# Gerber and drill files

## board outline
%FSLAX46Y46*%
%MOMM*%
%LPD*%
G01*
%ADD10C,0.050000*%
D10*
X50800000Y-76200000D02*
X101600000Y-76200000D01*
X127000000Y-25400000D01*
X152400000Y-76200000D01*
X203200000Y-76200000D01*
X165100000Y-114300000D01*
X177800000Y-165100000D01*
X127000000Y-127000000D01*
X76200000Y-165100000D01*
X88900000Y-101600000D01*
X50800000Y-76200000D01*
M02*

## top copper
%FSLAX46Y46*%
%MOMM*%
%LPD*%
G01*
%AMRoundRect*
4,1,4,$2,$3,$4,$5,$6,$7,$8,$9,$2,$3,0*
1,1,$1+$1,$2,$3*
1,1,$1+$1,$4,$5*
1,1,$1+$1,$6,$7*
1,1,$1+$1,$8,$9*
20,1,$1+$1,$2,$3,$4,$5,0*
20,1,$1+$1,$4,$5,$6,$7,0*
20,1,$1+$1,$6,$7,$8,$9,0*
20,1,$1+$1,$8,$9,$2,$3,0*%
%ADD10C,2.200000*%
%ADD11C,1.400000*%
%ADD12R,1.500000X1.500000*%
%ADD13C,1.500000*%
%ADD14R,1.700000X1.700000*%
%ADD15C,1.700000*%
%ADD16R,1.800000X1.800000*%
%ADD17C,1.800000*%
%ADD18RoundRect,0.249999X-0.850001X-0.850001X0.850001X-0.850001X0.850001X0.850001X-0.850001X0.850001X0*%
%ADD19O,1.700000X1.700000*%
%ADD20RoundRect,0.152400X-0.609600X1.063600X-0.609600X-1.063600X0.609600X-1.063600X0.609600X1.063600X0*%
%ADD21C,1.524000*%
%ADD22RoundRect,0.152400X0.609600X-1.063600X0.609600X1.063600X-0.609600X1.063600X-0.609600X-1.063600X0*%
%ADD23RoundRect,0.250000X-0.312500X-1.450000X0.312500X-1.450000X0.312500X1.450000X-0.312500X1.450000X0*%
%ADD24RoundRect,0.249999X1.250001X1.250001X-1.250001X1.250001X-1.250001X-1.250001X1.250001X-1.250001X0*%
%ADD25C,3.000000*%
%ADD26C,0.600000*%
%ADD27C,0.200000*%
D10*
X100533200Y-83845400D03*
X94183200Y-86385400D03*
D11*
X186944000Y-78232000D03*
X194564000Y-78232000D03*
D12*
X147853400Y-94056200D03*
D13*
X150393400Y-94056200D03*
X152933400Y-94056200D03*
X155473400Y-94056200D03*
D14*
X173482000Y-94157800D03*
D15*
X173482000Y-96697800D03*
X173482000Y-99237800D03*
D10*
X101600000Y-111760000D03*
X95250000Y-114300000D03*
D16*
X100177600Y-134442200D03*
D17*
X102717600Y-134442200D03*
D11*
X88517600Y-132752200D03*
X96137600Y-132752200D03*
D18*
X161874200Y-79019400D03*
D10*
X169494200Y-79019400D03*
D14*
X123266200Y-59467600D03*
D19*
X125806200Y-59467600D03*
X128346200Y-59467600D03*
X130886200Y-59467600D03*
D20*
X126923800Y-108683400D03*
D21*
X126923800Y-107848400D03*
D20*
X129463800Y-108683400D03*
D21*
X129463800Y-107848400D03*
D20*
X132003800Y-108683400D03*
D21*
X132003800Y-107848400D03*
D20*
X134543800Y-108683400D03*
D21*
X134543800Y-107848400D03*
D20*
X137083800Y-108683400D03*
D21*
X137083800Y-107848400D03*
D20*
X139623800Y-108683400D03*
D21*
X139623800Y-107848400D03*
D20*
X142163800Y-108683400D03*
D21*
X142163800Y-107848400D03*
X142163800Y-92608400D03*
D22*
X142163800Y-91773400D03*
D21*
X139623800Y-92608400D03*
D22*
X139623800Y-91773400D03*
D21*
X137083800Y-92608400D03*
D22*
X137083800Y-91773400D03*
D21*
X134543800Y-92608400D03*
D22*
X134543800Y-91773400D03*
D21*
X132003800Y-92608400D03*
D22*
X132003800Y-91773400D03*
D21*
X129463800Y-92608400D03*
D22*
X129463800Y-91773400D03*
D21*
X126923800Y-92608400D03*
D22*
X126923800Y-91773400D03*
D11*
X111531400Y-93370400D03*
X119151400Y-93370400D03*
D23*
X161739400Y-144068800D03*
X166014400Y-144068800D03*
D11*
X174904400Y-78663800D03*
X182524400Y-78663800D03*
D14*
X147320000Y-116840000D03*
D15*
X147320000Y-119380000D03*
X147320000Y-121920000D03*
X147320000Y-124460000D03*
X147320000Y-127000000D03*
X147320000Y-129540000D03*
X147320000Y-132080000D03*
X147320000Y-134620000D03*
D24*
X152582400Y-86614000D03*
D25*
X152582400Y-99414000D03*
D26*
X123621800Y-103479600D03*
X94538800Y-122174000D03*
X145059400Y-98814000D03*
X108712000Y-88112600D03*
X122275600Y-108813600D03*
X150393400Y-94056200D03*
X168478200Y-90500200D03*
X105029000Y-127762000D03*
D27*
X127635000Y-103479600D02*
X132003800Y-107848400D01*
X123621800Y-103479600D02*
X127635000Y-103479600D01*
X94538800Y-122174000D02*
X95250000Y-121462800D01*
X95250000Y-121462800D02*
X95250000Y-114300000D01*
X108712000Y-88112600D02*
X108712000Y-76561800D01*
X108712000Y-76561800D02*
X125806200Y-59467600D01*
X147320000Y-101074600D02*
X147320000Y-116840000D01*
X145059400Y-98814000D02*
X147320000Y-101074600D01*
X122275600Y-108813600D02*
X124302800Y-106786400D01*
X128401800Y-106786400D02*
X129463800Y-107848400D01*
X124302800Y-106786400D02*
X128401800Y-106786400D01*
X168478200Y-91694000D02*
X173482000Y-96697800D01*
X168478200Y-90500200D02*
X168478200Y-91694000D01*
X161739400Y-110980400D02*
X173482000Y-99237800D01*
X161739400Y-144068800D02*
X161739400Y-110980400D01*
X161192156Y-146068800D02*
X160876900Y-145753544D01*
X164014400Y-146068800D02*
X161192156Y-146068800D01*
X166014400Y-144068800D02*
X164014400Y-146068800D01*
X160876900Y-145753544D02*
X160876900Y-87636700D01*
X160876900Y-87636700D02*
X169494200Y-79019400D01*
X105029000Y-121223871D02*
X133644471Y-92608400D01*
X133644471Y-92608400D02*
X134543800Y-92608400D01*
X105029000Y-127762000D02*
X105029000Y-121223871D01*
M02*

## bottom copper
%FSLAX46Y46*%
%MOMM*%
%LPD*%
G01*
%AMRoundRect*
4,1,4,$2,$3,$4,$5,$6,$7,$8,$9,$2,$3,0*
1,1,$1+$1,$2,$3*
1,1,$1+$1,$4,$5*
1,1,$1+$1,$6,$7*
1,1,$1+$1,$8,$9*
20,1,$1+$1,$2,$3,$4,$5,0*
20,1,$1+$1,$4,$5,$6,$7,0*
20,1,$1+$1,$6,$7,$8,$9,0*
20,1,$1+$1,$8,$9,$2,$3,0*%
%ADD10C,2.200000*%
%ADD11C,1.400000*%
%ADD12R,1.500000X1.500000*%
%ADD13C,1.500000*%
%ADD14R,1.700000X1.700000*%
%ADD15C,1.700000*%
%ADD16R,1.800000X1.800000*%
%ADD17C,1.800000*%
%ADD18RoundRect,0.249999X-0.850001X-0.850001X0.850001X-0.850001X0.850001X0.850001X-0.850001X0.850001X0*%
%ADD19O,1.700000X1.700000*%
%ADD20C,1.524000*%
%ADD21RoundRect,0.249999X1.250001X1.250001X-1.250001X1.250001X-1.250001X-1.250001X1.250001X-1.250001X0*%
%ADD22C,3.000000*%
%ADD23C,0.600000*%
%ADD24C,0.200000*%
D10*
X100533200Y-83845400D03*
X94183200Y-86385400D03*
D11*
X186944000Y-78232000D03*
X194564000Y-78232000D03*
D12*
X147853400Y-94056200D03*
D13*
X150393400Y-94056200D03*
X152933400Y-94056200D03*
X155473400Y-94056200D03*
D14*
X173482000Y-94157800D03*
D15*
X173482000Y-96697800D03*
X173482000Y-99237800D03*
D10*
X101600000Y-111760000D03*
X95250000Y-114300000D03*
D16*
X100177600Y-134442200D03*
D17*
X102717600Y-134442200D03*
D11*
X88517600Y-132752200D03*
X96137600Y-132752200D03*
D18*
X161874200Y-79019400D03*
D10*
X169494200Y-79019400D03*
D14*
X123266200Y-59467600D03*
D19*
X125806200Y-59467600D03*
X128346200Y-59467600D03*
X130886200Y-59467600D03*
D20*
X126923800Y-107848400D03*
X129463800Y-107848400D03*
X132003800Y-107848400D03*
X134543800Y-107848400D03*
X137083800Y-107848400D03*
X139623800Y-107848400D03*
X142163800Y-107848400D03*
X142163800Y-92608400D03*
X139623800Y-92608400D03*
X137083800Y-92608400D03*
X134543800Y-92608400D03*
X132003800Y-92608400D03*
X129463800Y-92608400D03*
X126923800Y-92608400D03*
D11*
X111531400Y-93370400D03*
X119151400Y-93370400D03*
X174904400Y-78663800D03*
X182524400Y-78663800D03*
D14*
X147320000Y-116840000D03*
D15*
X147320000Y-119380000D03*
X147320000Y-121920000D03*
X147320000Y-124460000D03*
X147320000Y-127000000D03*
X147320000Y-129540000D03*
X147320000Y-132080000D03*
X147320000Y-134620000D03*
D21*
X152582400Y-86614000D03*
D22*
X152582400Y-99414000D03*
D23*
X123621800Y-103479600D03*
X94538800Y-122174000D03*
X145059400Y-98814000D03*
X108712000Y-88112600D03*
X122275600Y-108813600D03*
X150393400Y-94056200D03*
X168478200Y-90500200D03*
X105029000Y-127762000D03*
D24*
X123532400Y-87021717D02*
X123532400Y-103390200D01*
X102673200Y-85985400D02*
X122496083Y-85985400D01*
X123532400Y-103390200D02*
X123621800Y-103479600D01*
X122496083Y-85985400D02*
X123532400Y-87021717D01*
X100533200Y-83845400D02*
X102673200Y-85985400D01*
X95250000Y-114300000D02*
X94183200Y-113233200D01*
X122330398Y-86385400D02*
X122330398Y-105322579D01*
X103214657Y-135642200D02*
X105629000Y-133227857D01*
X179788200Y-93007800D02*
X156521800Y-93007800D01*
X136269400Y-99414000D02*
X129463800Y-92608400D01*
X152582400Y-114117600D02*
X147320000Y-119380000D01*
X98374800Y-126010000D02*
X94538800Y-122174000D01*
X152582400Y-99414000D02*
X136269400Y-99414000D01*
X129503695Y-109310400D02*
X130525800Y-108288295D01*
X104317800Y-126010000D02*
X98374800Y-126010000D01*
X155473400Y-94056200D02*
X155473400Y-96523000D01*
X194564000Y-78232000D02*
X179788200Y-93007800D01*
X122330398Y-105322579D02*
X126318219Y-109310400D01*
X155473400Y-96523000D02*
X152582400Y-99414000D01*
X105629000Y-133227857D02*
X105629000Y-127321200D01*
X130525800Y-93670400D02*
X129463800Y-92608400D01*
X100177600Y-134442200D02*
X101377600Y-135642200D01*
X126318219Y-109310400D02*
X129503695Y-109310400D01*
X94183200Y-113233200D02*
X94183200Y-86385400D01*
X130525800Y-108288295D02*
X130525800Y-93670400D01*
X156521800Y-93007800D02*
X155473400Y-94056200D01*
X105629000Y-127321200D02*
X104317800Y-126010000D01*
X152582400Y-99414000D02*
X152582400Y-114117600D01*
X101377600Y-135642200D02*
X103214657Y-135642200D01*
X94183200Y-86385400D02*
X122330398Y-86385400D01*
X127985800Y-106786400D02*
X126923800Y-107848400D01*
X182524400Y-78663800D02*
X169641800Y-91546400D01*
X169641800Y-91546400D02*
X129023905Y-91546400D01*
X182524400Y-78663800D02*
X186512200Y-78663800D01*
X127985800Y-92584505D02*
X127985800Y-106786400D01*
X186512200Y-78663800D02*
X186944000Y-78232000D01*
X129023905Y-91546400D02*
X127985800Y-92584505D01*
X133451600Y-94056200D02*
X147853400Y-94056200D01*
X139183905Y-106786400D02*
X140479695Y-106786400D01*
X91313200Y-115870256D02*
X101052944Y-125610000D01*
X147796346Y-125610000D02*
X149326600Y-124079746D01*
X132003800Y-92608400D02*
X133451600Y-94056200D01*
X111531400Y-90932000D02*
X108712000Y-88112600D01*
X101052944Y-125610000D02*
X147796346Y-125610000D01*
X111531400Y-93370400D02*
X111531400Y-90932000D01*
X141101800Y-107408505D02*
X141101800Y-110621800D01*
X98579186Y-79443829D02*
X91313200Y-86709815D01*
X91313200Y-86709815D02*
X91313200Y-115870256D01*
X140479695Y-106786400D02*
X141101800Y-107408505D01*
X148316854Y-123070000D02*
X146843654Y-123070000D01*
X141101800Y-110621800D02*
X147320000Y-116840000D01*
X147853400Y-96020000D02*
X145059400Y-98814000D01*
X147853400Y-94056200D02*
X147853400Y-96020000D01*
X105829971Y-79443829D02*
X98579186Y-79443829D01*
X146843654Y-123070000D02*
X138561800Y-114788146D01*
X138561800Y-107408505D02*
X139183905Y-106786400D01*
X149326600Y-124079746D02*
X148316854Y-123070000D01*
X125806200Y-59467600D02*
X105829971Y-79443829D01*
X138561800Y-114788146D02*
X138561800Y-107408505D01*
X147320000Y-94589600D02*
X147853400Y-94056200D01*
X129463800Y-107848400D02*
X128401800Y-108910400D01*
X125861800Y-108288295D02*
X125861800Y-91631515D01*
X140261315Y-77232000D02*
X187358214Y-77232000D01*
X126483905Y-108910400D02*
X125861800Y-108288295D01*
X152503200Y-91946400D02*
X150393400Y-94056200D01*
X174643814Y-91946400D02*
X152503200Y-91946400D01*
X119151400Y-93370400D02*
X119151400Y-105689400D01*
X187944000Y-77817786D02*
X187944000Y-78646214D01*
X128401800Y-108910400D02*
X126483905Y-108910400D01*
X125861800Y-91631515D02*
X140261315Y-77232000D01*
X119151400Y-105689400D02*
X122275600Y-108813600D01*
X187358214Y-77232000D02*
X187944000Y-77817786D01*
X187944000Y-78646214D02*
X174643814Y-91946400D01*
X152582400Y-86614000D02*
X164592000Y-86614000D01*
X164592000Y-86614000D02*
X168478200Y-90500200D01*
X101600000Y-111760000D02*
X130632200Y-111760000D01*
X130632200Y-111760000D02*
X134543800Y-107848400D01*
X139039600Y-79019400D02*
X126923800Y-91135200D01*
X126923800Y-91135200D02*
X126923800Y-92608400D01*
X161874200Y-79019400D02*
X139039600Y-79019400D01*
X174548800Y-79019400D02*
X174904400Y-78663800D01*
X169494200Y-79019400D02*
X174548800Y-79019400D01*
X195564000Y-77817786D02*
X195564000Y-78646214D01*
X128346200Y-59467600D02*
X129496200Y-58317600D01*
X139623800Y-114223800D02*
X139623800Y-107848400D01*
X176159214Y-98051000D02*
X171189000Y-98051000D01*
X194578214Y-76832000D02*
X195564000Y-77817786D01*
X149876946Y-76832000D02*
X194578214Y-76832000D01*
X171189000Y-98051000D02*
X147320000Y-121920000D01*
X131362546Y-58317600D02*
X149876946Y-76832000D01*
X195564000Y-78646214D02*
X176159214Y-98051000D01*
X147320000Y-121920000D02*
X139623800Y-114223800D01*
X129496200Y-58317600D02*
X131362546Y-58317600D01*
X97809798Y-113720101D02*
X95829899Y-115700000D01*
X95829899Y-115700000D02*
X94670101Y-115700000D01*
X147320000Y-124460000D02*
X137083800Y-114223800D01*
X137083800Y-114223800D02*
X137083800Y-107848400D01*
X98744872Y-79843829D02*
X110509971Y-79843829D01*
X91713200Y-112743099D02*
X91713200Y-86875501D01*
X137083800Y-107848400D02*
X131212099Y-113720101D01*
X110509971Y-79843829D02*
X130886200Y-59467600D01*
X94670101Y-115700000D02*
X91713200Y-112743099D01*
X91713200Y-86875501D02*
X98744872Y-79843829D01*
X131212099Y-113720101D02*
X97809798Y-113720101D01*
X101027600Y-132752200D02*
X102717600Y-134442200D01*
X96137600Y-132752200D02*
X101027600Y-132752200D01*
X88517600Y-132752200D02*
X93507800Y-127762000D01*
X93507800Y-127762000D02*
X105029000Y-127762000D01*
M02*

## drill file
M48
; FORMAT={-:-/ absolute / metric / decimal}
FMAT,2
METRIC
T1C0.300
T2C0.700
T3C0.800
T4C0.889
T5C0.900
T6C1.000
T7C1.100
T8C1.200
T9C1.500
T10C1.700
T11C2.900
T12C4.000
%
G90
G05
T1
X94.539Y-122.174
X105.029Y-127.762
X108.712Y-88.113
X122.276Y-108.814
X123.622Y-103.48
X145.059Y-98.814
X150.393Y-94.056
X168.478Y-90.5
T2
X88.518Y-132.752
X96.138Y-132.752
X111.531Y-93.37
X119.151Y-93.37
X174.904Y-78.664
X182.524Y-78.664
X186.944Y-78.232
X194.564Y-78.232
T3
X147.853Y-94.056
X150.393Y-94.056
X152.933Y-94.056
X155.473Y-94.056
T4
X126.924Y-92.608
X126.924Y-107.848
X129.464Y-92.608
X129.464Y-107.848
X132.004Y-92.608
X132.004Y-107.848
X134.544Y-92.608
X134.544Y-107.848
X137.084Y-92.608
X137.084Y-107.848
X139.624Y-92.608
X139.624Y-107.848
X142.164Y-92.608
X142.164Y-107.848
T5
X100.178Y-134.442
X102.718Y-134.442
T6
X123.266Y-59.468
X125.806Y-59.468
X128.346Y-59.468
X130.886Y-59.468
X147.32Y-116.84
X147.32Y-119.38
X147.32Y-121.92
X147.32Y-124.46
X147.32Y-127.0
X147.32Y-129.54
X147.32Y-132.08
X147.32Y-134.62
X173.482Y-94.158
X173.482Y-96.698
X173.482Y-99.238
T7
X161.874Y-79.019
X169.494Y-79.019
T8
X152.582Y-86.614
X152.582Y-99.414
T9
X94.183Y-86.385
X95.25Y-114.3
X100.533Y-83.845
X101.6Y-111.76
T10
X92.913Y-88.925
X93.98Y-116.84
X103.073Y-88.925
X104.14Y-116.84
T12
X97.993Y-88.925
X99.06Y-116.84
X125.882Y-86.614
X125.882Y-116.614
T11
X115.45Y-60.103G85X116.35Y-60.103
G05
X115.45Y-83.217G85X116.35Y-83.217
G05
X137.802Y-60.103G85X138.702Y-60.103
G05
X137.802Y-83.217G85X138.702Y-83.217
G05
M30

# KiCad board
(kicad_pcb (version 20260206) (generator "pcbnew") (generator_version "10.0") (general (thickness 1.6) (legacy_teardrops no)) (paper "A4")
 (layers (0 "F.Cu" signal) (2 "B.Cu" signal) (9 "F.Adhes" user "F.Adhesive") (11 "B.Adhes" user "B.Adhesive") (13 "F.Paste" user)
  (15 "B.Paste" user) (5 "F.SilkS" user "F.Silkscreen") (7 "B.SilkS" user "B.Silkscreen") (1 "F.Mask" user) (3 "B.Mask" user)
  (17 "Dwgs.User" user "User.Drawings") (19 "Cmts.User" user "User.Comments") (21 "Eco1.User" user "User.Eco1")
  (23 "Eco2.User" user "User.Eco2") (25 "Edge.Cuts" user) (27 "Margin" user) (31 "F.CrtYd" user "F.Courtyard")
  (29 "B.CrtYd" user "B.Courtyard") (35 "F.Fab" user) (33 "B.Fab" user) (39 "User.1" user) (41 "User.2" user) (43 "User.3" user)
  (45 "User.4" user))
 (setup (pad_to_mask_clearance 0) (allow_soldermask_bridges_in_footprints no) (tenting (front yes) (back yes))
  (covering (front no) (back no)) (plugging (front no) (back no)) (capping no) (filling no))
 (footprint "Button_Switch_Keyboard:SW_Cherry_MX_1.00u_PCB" (layer "F.Cu") (at 100.5332 83.8454)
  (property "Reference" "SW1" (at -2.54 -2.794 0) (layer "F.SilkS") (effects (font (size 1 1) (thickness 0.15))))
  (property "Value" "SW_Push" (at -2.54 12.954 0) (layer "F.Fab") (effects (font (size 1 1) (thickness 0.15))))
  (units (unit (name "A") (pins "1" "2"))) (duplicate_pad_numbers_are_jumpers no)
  (pad "" np_thru_hole circle (at -7.62 5.08) (size 1.7 1.7) (drill 1.7) (layers "*.Cu" "*.Mask"))
  (pad "" np_thru_hole circle (at -2.54 5.08) (size 4 4) (drill 4) (layers "*.Cu" "*.Mask"))
  (pad "" np_thru_hole circle (at 2.54 5.08) (size 1.7 1.7) (drill 1.7) (layers "*.Cu" "*.Mask"))
  (pad "1" thru_hole circle (at 0 0) (size 2.2 2.2) (drill 1.5) (layers "*.Cu" "*.Mask") (remove_unused_layers no) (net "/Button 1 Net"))
  (pad "2" thru_hole circle (at -6.35 2.54) (size 2.2 2.2) (drill 1.5) (layers "*.Cu" "*.Mask") (remove_unused_layers no) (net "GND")))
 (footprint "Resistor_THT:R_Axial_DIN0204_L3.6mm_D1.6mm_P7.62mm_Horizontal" (layer "F.Cu") (at 186.944 78.232)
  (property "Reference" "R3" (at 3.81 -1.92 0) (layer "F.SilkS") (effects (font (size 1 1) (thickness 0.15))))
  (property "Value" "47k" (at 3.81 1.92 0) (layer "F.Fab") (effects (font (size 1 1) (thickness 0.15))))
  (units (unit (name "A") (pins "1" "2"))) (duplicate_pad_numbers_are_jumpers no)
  (pad "1" thru_hole circle (at 0 0) (size 1.4 1.4) (drill 0.7) (layers "*.Cu" "*.Mask") (remove_unused_layers no) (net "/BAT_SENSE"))
  (pad "2" thru_hole circle (at 7.62 0) (size 1.4 1.4) (drill 0.7) (layers "*.Cu" "*.Mask") (remove_unused_layers no) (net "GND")))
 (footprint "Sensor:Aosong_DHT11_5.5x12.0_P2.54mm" (layer "F.Cu") (at 147.8534 94.0562 90)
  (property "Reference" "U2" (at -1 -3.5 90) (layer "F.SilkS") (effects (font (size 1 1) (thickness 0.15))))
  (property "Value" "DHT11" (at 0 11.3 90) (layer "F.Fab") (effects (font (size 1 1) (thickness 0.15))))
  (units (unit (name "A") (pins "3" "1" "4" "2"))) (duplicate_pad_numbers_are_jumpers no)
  (pad "1" thru_hole rect (at 0 0 90) (size 1.5 1.5) (drill 0.8) (layers "*.Cu" "*.Mask") (remove_unused_layers no) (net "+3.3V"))
  (pad "2" thru_hole circle (at 0 2.54 90) (size 1.5 1.5) (drill 0.8) (layers "*.Cu" "*.Mask") (remove_unused_layers no) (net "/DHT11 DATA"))
  (pad "3" thru_hole circle (at 0 5.08 90) (size 1.5 1.5) (drill 0.8) (layers "*.Cu" "*.Mask") (remove_unused_layers no)
   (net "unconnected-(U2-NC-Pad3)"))
  (pad "4" thru_hole circle (at 0 7.62 90) (size 1.5 1.5) (drill 0.8) (layers "*.Cu" "*.Mask") (remove_unused_layers no) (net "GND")))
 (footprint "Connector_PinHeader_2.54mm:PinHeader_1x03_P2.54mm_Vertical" (layer "F.Cu") (at 173.482 94.1578)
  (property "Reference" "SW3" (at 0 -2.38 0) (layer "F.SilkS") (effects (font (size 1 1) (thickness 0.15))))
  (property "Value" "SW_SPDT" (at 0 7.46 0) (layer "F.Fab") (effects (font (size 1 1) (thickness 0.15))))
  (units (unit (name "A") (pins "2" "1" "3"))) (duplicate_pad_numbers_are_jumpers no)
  (pad "1" thru_hole rect (at 0 0) (size 1.7 1.7) (drill 1) (layers "*.Cu" "*.Mask") (remove_unused_layers no)
   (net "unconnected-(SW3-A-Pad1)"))
  (pad "2" thru_hole circle (at 0 2.54) (size 1.7 1.7) (drill 1) (layers "*.Cu" "*.Mask") (remove_unused_layers no) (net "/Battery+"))
  (pad "3" thru_hole circle (at 0 5.08) (size 1.7 1.7) (drill 1) (layers "*.Cu" "*.Mask") (remove_unused_layers no) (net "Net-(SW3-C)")))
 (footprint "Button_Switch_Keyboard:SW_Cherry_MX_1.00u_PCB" (layer "F.Cu") (at 101.6 111.76)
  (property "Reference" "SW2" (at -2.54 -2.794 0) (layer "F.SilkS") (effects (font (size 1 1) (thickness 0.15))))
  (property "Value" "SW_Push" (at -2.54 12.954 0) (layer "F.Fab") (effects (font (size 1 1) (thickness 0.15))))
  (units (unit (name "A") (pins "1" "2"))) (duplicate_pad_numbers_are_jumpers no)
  (pad "" np_thru_hole circle (at -7.62 5.08) (size 1.7 1.7) (drill 1.7) (layers "*.Cu" "*.Mask"))
  (pad "" np_thru_hole circle (at -2.54 5.08) (size 4 4) (drill 4) (layers "*.Cu" "*.Mask"))
  (pad "" np_thru_hole circle (at 2.54 5.08) (size 1.7 1.7) (drill 1.7) (layers "*.Cu" "*.Mask"))
  (pad "1" thru_hole circle (at 0 0) (size 2.2 2.2) (drill 1.5) (layers "*.Cu" "*.Mask") (remove_unused_layers no) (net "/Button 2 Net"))
  (pad "2" thru_hole circle (at -6.35 2.54) (size 2.2 2.2) (drill 1.5) (layers "*.Cu" "*.Mask") (remove_unused_layers no) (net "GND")))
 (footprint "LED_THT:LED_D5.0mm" (layer "F.Cu") (at 100.1776 134.4422)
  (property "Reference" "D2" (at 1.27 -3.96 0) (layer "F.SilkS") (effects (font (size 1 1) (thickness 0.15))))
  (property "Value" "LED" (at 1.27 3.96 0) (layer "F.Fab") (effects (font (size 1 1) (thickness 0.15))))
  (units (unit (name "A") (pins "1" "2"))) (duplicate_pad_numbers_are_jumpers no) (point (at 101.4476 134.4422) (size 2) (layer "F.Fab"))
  (pad "1" thru_hole rect (at 0 0) (size 1.8 1.8) (drill 0.9) (layers "*.Cu" "*.Mask") (remove_unused_layers no) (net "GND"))
  (pad "2" thru_hole circle (at 2.54 0) (size 1.8 1.8) (drill 0.9) (layers "*.Cu" "*.Mask") (remove_unused_layers no) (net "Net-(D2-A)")))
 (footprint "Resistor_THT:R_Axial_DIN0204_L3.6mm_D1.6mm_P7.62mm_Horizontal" (layer "F.Cu") (at 88.5176 132.7522)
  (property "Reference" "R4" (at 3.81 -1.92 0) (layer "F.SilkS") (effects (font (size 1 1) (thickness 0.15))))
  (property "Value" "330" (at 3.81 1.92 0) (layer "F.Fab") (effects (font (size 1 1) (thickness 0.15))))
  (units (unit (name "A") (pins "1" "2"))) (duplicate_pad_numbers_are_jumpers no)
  (pad "1" thru_hole circle (at 0 0) (size 1.4 1.4) (drill 0.7) (layers "*.Cu" "*.Mask") (remove_unused_layers no) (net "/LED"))
  (pad "2" thru_hole circle (at 7.62 0) (size 1.4 1.4) (drill 0.7) (layers "*.Cu" "*.Mask") (remove_unused_layers no) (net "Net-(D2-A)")))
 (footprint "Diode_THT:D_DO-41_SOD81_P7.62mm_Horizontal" (layer "F.Cu") (at 161.8742 79.0194)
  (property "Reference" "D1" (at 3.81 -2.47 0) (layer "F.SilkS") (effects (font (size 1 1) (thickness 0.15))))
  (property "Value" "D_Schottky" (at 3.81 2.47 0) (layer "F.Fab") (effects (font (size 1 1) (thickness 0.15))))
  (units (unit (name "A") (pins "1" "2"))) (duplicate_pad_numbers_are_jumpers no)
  (pad "1" thru_hole roundrect (at 0 0) (size 2.2 2.2) (drill 1.1) (layers "*.Cu" "*.Mask") (remove_unused_layers no)
   (roundrect_rratio 0.113636) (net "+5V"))
  (pad "2" thru_hole circle (at 7.62 0) (size 2.2 2.2) (drill 1.1) (layers "*.Cu" "*.Mask") (remove_unused_layers no) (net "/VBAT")))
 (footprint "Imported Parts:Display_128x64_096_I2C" (layer "F.Cu") (at 127.0762 59.4676)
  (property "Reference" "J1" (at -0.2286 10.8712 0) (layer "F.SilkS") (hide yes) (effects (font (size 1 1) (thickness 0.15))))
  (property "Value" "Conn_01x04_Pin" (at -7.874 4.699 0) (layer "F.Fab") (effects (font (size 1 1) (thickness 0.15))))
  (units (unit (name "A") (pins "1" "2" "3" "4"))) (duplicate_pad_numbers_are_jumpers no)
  (pad "" np_thru_hole oval (at -11.176 0.635) (size 3.8 2.9) (drill oval 3.8 2.9) (layers "*.Cu" "*.Mask"))
  (pad "" np_thru_hole oval (at -11.176 23.749) (size 3.8 2.9) (drill oval 3.8 2.9) (layers "*.Cu" "*.Mask"))
  (pad "" np_thru_hole oval (at 11.176 0.635) (size 3.8 2.9) (drill oval 3.8 2.9) (layers "*.Cu" "*.Mask"))
  (pad "" np_thru_hole oval (at 11.176 23.749) (size 3.8 2.9) (drill oval 3.8 2.9) (layers "*.Cu" "*.Mask"))
  (pad "1" thru_hole rect (at -3.81 0 90) (size 1.7 1.7) (drill 1) (layers "*.Cu" "*.Mask") (remove_unused_layers no) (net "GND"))
  (pad "2" thru_hole oval (at -1.27 0 90) (size 1.7 1.7) (drill 1) (layers "*.Cu" "*.Mask") (remove_unused_layers no) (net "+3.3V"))
  (pad "3" thru_hole oval (at 1.27 0 90) (size 1.7 1.7) (drill 1) (layers "*.Cu" "*.Mask") (remove_unused_layers no) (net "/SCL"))
  (pad "4" thru_hole oval (at 3.81 0 90) (size 1.7 1.7) (drill 1) (layers "*.Cu" "*.Mask") (remove_unused_layers no) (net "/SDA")))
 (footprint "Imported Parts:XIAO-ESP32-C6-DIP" (layer "F.Cu") (at 134.5438 100.2284 180)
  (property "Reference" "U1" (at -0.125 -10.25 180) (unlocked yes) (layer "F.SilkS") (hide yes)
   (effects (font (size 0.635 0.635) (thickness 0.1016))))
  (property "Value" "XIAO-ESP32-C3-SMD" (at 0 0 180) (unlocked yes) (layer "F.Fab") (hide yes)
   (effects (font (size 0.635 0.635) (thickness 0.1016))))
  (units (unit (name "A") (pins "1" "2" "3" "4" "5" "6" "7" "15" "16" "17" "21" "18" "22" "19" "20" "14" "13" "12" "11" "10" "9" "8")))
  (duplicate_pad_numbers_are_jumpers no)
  (pad "1" smd roundrect (at 7.62 -8.455 270) (size 2.432 1.524) (layers "F.Cu" "F.Mask") (roundrect_rratio 0.1) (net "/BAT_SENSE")
   (thermal_bridge_angle 45))
  (pad "1" thru_hole circle (at 7.62 -7.62 270) (size 1.524 1.524) (drill 0.889) (layers "*.Cu" "*.Mask") (remove_unused_layers no)
   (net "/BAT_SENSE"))
  (pad "2" smd roundrect (at 5.08 -8.455 270) (size 2.432 1.524) (layers "F.Cu" "F.Mask") (roundrect_rratio 0.1) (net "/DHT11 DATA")
   (thermal_bridge_angle 45))
  (pad "2" thru_hole circle (at 5.08 -7.62 270) (size 1.524 1.524) (drill 0.889) (layers "*.Cu" "*.Mask") (remove_unused_layers no)
   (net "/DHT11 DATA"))
  (pad "3" smd roundrect (at 2.54 -8.455 270) (size 2.432 1.524) (layers "F.Cu" "F.Mask") (roundrect_rratio 0.1) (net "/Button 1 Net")
   (thermal_bridge_angle 45))
  (pad "3" thru_hole circle (at 2.54 -7.62 270) (size 1.524 1.524) (drill 0.889) (layers "*.Cu" "*.Mask") (remove_unused_layers no)
   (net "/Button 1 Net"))
  (pad "4" smd roundrect (at 0 -8.455 270) (size 2.432 1.524) (layers "F.Cu" "F.Mask") (roundrect_rratio 0.1) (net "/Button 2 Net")
   (thermal_bridge_angle 45))
  (pad "4" thru_hole circle (at 0 -7.62 270) (size 1.524 1.524) (drill 0.889) (layers "*.Cu" "*.Mask") (remove_unused_layers no)
   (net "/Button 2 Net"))
  (pad "5" smd roundrect (at -2.54 -8.455 270) (size 2.432 1.524) (layers "F.Cu" "F.Mask") (roundrect_rratio 0.1) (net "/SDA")
   (thermal_bridge_angle 45))
  (pad "5" thru_hole circle (at -2.54 -7.62 270) (size 1.524 1.524) (drill 0.889) (layers "*.Cu" "*.Mask") (remove_unused_layers no)
   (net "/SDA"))
  (pad "6" smd roundrect (at -5.08 -8.455 270) (size 2.432 1.524) (layers "F.Cu" "F.Mask") (roundrect_rratio 0.1) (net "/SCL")
   (thermal_bridge_angle 45))
  (pad "6" thru_hole circle (at -5.08 -7.62 270) (size 1.524 1.524) (drill 0.889) (layers "*.Cu" "*.Mask") (remove_unused_layers no)
   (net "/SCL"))
  (pad "7" smd roundrect (at -7.62 -8.455 270) (size 2.432 1.524) (layers "F.Cu" "F.Mask") (roundrect_rratio 0.1)
   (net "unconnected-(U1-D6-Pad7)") (thermal_bridge_angle 45))
  (pad "7" thru_hole circle (at -7.62 -7.62 270) (size 1.524 1.524) (drill 0.889) (layers "*.Cu" "*.Mask") (remove_unused_layers no)
   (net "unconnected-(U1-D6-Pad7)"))
  (pad "8" thru_hole circle (at -7.62 7.62 90) (size 1.524 1.524) (drill 0.889) (layers "*.Cu" "*.Mask") (remove_unused_layers no)
   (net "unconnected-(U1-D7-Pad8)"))
  (pad "8" smd roundrect (at -7.62 8.455 90) (size 2.432 1.524) (layers "F.Cu" "F.Mask") (roundrect_rratio 0.1)
   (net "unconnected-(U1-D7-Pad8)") (thermal_bridge_angle 45))
  (pad "9" thru_hole circle (at -5.08 7.62 90) (size 1.524 1.524) (drill 0.889) (layers "*.Cu" "*.Mask") (remove_unused_layers no)
   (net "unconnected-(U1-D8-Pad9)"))
  (pad "9" smd roundrect (at -5.08 8.455 90) (size 2.432 1.524) (layers "F.Cu" "F.Mask") (roundrect_rratio 0.1)
   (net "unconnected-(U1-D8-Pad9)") (thermal_bridge_angle 45))
  (pad "10" thru_hole circle (at -2.54 7.62 90) (size 1.524 1.524) (drill 0.889) (layers "*.Cu" "*.Mask") (remove_unused_layers no)
   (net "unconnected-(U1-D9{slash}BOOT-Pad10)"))
  (pad "10" smd roundrect (at -2.54 8.455 90) (size 2.432 1.524) (layers "F.Cu" "F.Mask") (roundrect_rratio 0.1)
   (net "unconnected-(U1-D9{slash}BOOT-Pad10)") (thermal_bridge_angle 45))
  (pad "11" thru_hole circle (at 0 7.62 90) (size 1.524 1.524) (drill 0.889) (layers "*.Cu" "*.Mask") (remove_unused_layers no) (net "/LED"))
  (pad "11" smd roundrect (at 0 8.455 90) (size 2.432 1.524) (layers "F.Cu" "F.Mask") (roundrect_rratio 0.1) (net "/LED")
   (thermal_bridge_angle 45))
  (pad "12" thru_hole circle (at 2.54 7.62 90) (size 1.524 1.524) (drill 0.889) (layers "*.Cu" "*.Mask") (remove_unused_layers no)
   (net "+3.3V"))
  (pad "12" smd roundrect (at 2.54 8.455 90) (size 2.432 1.524) (layers "F.Cu" "F.Mask") (roundrect_rratio 0.1) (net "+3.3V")
   (thermal_bridge_angle 45))
  (pad "13" thru_hole circle (at 5.08 7.62 90) (size 1.524 1.524) (drill 0.889) (layers "*.Cu" "*.Mask") (remove_unused_layers no)
   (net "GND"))
  (pad "13" smd roundrect (at 5.08 8.455 90) (size 2.432 1.524) (layers "F.Cu" "F.Mask") (roundrect_rratio 0.1) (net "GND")
   (thermal_bridge_angle 45))
  (pad "14" thru_hole circle (at 7.62 7.62 90) (size 1.524 1.524) (drill 0.889) (layers "*.Cu" "*.Mask") (remove_unused_layers no)
   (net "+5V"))
  (pad "14" smd roundrect (at 7.62 8.455 90) (size 2.432 1.524) (layers "F.Cu" "F.Mask") (roundrect_rratio 0.1) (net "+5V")
   (thermal_bridge_angle 45)))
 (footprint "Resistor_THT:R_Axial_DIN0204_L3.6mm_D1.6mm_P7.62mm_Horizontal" (layer "F.Cu") (at 111.5314 93.3704)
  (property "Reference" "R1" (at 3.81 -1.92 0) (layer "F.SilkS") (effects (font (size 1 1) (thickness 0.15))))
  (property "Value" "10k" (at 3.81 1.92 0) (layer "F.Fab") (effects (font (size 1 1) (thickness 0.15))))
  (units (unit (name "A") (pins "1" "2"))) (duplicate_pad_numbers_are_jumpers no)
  (pad "1" thru_hole circle (at 0 0) (size 1.4 1.4) (drill 0.7) (layers "*.Cu" "*.Mask") (remove_unused_layers no) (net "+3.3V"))
  (pad "2" thru_hole circle (at 7.62 0) (size 1.4 1.4) (drill 0.7) (layers "*.Cu" "*.Mask") (remove_unused_layers no) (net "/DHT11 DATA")))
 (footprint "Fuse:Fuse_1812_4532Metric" (layer "F.Cu") (at 163.8769 144.0688)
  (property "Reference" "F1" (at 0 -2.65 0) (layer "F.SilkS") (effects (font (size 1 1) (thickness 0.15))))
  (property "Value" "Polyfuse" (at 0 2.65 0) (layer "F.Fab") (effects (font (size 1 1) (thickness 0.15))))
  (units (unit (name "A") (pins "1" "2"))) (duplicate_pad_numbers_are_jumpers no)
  (pad "1" smd roundrect (at -2.1375 0) (size 1.125 3.4) (layers "F.Cu" "F.Mask" "F.Paste") (roundrect_rratio 0.222222) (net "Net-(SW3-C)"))
  (pad "2" smd roundrect (at 2.1375 0) (size 1.125 3.4) (layers "F.Cu" "F.Mask" "F.Paste") (roundrect_rratio 0.222222) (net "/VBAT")))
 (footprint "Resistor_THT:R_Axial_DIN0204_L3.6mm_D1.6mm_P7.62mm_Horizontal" (layer "F.Cu") (at 174.9044 78.6638)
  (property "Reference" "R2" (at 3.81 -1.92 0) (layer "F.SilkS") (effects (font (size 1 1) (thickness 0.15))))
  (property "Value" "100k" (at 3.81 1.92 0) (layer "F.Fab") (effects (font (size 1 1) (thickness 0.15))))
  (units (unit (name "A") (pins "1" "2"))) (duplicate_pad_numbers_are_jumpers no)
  (pad "1" thru_hole circle (at 0 0) (size 1.4 1.4) (drill 0.7) (layers "*.Cu" "*.Mask") (remove_unused_layers no) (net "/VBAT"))
  (pad "2" thru_hole circle (at 7.62 0) (size 1.4 1.4) (drill 0.7) (layers "*.Cu" "*.Mask") (remove_unused_layers no) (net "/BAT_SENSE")))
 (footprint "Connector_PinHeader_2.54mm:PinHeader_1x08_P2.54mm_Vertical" (layer "F.Cu") (at 147.32 116.84)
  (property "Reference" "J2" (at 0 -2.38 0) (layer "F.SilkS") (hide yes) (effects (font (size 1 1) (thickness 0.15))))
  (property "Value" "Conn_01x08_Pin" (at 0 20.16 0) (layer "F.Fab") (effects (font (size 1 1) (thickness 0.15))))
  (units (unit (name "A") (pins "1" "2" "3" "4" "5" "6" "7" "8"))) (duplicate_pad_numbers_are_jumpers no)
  (pad "1" thru_hole rect (at 0 0) (size 1.7 1.7) (drill 1) (layers "*.Cu" "*.Mask") (remove_unused_layers no) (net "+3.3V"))
  (pad "2" thru_hole circle (at 0 2.54) (size 1.7 1.7) (drill 1) (layers "*.Cu" "*.Mask") (remove_unused_layers no) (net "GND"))
  (pad "3" thru_hole circle (at 0 5.08) (size 1.7 1.7) (drill 1) (layers "*.Cu" "*.Mask") (remove_unused_layers no) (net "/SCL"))
  (pad "4" thru_hole circle (at 0 7.62) (size 1.7 1.7) (drill 1) (layers "*.Cu" "*.Mask") (remove_unused_layers no) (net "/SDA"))
  (pad "5" thru_hole circle (at 0 10.16) (size 1.7 1.7) (drill 1) (layers "*.Cu" "*.Mask") (remove_unused_layers no)
   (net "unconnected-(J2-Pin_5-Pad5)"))
  (pad "6" thru_hole circle (at 0 12.7) (size 1.7 1.7) (drill 1) (layers "*.Cu" "*.Mask") (remove_unused_layers no)
   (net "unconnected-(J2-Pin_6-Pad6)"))
  (pad "7" thru_hole circle (at 0 15.24) (size 1.7 1.7) (drill 1) (layers "*.Cu" "*.Mask") (remove_unused_layers no)
   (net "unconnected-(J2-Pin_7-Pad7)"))
  (pad "8" thru_hole circle (at 0 17.78) (size 1.7 1.7) (drill 1) (layers "*.Cu" "*.Mask") (remove_unused_layers no)
   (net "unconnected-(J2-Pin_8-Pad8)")))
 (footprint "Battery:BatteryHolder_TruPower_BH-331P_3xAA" (layer "B.Cu") (at 152.5824 86.614 180)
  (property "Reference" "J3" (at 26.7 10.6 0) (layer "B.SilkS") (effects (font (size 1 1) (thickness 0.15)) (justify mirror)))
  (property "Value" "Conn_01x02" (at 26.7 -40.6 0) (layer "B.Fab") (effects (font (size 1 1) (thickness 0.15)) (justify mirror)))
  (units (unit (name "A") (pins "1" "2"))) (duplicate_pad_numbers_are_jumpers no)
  (pad "" np_thru_hole circle (at 26.7 -30 180) (size 4 4) (drill 4) (layers "*.Cu" "*.Mask"))
  (pad "" np_thru_hole circle (at 26.7 0 180) (size 4 4) (drill 4) (layers "*.Cu" "*.Mask"))
  (pad "1" thru_hole roundrect (at 0 0 180) (size 3 3) (drill 1.2) (layers "*.Cu" "*.Mask") (remove_unused_layers no)
   (roundrect_rratio 0.083333) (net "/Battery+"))
  (pad "2" thru_hole circle (at 0 -12.8 180) (size 3 3) (drill 1.2) (layers "*.Cu" "*.Mask") (remove_unused_layers no) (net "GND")))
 (gr_poly
  (pts (xy 50.8 76.2) (xy 101.6 76.2) (xy 127 25.4) (xy 152.4 76.2) (xy 203.2 76.2) (xy 165.1 114.3) (xy 177.8 165.1) (xy 127 127)
   (xy 76.2 165.1) (xy 88.9 101.6))
  (stroke (width 0.05) (type solid)) (fill no) (layer "Edge.Cuts"))
 (segment (start 127.635 103.4796) (end 132.0038 107.8484) (width 0.2) (layer "F.Cu") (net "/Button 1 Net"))
 (segment (start 123.6218 103.4796) (end 127.635 103.4796) (width 0.2) (layer "F.Cu") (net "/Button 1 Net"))
 (via (at 123.6218 103.4796) (size 0.6) (drill 0.3) (layers "F.Cu" "B.Cu") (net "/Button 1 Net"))
 (segment (start 123.5324 87.021717) (end 123.5324 103.3902) (width 0.2) (layer "B.Cu") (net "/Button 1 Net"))
 (segment (start 102.6732 85.9854) (end 122.496083 85.9854) (width 0.2) (layer "B.Cu") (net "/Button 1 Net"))
 (segment (start 123.5324 103.3902) (end 123.6218 103.4796) (width 0.2) (layer "B.Cu") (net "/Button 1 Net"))
 (segment (start 122.496083 85.9854) (end 123.5324 87.021717) (width 0.2) (layer "B.Cu") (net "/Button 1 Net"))
 (segment (start 100.5332 83.8454) (end 102.6732 85.9854) (width 0.2) (layer "B.Cu") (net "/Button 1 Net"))
 (segment (start 94.5388 122.174) (end 95.25 121.4628) (width 0.2) (layer "F.Cu") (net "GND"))
 (segment (start 95.25 121.4628) (end 95.25 114.3) (width 0.2) (layer "F.Cu") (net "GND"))
 (via (at 94.5388 122.174) (size 0.6) (drill 0.3) (layers "F.Cu" "B.Cu") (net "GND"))
 (segment (start 95.25 114.3) (end 94.1832 113.2332) (width 0.2) (layer "B.Cu") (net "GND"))
 (segment (start 122.330398 86.3854) (end 122.330398 105.322579) (width 0.2) (layer "B.Cu") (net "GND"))
 (segment (start 103.214657 135.6422) (end 105.629 133.227857) (width 0.2) (layer "B.Cu") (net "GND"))
 (segment (start 179.7882 93.0078) (end 156.5218 93.0078) (width 0.2) (layer "B.Cu") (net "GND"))
 (segment (start 136.2694 99.414) (end 129.4638 92.6084) (width 0.2) (layer "B.Cu") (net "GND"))
 (segment (start 152.5824 114.1176) (end 147.32 119.38) (width 0.2) (layer "B.Cu") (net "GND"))
 (segment (start 98.3748 126.01) (end 94.5388 122.174) (width 0.2) (layer "B.Cu") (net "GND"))
 (segment (start 152.5824 99.414) (end 136.2694 99.414) (width 0.2) (layer "B.Cu") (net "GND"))
 (segment (start 129.503695 109.3104) (end 130.5258 108.288295) (width 0.2) (layer "B.Cu") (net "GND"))
 (segment (start 104.3178 126.01) (end 98.3748 126.01) (width 0.2) (layer "B.Cu") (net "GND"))
 (segment (start 155.4734 94.0562) (end 155.4734 96.523) (width 0.2) (layer "B.Cu") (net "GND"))
 (segment (start 194.564 78.232) (end 179.7882 93.0078) (width 0.2) (layer "B.Cu") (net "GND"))
 (segment (start 122.330398 105.322579) (end 126.318219 109.3104) (width 0.2) (layer "B.Cu") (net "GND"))
 (segment (start 155.4734 96.523) (end 152.5824 99.414) (width 0.2) (layer "B.Cu") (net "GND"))
 (segment (start 105.629 133.227857) (end 105.629 127.3212) (width 0.2) (layer "B.Cu") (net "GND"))
 (segment (start 130.5258 93.6704) (end 129.4638 92.6084) (width 0.2) (layer "B.Cu") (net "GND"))
 (segment (start 100.1776 134.4422) (end 101.3776 135.6422) (width 0.2) (layer "B.Cu") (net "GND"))
 (segment (start 126.318219 109.3104) (end 129.503695 109.3104) (width 0.2) (layer "B.Cu") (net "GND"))
 (segment (start 94.1832 113.2332) (end 94.1832 86.3854) (width 0.2) (layer "B.Cu") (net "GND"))
 (segment (start 130.5258 108.288295) (end 130.5258 93.6704) (width 0.2) (layer "B.Cu") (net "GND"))
 (segment (start 156.5218 93.0078) (end 155.4734 94.0562) (width 0.2) (layer "B.Cu") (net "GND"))
 (segment (start 105.629 127.3212) (end 104.3178 126.01) (width 0.2) (layer "B.Cu") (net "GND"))
 (segment (start 152.5824 99.414) (end 152.5824 114.1176) (width 0.2) (layer "B.Cu") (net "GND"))
 (segment (start 101.3776 135.6422) (end 103.214657 135.6422) (width 0.2) (layer "B.Cu") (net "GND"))
 (segment (start 94.1832 86.3854) (end 122.330398 86.3854) (width 0.2) (layer "B.Cu") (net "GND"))
 (segment (start 127.9858 106.7864) (end 126.9238 107.8484) (width 0.2) (layer "B.Cu") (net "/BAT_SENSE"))
 (segment (start 182.5244 78.6638) (end 169.6418 91.5464) (width 0.2) (layer "B.Cu") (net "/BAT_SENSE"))
 (segment (start 169.6418 91.5464) (end 129.023905 91.5464) (width 0.2) (layer "B.Cu") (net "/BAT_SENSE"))
 (segment (start 182.5244 78.6638) (end 186.5122 78.6638) (width 0.2) (layer "B.Cu") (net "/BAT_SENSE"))
 (segment (start 127.9858 92.584505) (end 127.9858 106.7864) (width 0.2) (layer "B.Cu") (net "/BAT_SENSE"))
 (segment (start 186.5122 78.6638) (end 186.944 78.232) (width 0.2) (layer "B.Cu") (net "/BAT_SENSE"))
 (segment (start 129.023905 91.5464) (end 127.9858 92.584505) (width 0.2) (layer "B.Cu") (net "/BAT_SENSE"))
 (segment (start 108.712 88.1126) (end 108.712 76.5618) (width 0.2) (layer "F.Cu") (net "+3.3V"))
 (segment (start 108.712 76.5618) (end 125.8062 59.4676) (width 0.2) (layer "F.Cu") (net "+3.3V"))
 (segment (start 147.32 101.0746) (end 147.32 116.84) (width 0.2) (layer "F.Cu") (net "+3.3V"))
 (segment (start 145.0594 98.814) (end 147.32 101.0746) (width 0.2) (layer "F.Cu") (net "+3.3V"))
 (via (at 145.0594 98.814) (size 0.6) (drill 0.3) (layers "F.Cu" "B.Cu") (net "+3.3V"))
 (via (at 108.712 88.1126) (size 0.6) (drill 0.3) (layers "F.Cu" "B.Cu") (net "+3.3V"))
 (segment (start 133.4516 94.0562) (end 147.8534 94.0562) (width 0.2) (layer "B.Cu") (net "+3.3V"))
 (segment (start 139.183905 106.7864) (end 140.479695 106.7864) (width 0.2) (layer "B.Cu") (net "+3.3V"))
 (segment (start 91.3132 115.870256) (end 101.052944 125.61) (width 0.2) (layer "B.Cu") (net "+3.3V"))
 (segment (start 147.796346 125.61) (end 149.3266 124.079746) (width 0.2) (layer "B.Cu") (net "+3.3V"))
 (segment (start 132.0038 92.6084) (end 133.4516 94.0562) (width 0.2) (layer "B.Cu") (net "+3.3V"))
 (segment (start 111.5314 90.932) (end 108.712 88.1126) (width 0.2) (layer "B.Cu") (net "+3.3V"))
 (segment (start 101.052944 125.61) (end 147.796346 125.61) (width 0.2) (layer "B.Cu") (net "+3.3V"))
 (segment (start 111.5314 93.3704) (end 111.5314 90.932) (width 0.2) (layer "B.Cu") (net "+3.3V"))
 (segment (start 141.1018 107.408505) (end 141.1018 110.6218) (width 0.2) (layer "B.Cu") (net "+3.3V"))
 (segment (start 98.579186 79.443829) (end 91.3132 86.709815) (width 0.2) (layer "B.Cu") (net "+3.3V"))
 (segment (start 91.3132 86.709815) (end 91.3132 115.870256) (width 0.2) (layer "B.Cu") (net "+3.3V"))
 (segment (start 140.479695 106.7864) (end 141.1018 107.408505) (width 0.2) (layer "B.Cu") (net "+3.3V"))
 (segment (start 148.316854 123.07) (end 146.843654 123.07) (width 0.2) (layer "B.Cu") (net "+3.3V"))
 (segment (start 141.1018 110.6218) (end 147.32 116.84) (width 0.2) (layer "B.Cu") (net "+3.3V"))
 (segment (start 147.8534 96.02) (end 145.0594 98.814) (width 0.2) (layer "B.Cu") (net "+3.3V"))
 (segment (start 147.8534 94.0562) (end 147.8534 96.02) (width 0.2) (layer "B.Cu") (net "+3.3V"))
 (segment (start 105.829971 79.443829) (end 98.579186 79.443829) (width 0.2) (layer "B.Cu") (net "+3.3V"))
 (segment (start 146.843654 123.07) (end 138.5618 114.788146) (width 0.2) (layer "B.Cu") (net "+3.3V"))
 (segment (start 138.5618 107.408505) (end 139.183905 106.7864) (width 0.2) (layer "B.Cu") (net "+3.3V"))
 (segment (start 149.3266 124.079746) (end 148.316854 123.07) (width 0.2) (layer "B.Cu") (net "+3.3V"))
 (segment (start 125.8062 59.4676) (end 105.829971 79.443829) (width 0.2) (layer "B.Cu") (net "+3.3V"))
 (segment (start 138.5618 114.788146) (end 138.5618 107.408505) (width 0.2) (layer "B.Cu") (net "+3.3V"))
 (segment (start 147.32 94.5896) (end 147.8534 94.0562) (width 0.2) (layer "B.Cu") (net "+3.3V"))
 (segment (start 122.2756 108.8136) (end 124.3028 106.7864) (width 0.2) (layer "F.Cu") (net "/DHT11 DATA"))
 (segment (start 128.4018 106.7864) (end 129.4638 107.8484) (width 0.2) (layer "F.Cu") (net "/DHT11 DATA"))
 (segment (start 124.3028 106.7864) (end 128.4018 106.7864) (width 0.2) (layer "F.Cu") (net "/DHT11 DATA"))
 (via (at 122.2756 108.8136) (size 0.6) (drill 0.3) (layers "F.Cu" "B.Cu") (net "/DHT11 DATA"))
 (via (at 150.3934 94.0562) (size 0.6) (drill 0.3) (layers "F.Cu" "B.Cu") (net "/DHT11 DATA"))
 (segment (start 129.4638 107.8484) (end 128.4018 108.9104) (width 0.2) (layer "B.Cu") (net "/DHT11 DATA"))
 (segment (start 125.8618 108.288295) (end 125.8618 91.631515) (width 0.2) (layer "B.Cu") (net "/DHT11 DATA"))
 (segment (start 140.261315 77.232) (end 187.358214 77.232) (width 0.2) (layer "B.Cu") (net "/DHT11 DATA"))
 (segment (start 126.483905 108.9104) (end 125.8618 108.288295) (width 0.2) (layer "B.Cu") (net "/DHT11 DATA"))
 (segment (start 152.5032 91.9464) (end 150.3934 94.0562) (width 0.2) (layer "B.Cu") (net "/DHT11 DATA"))
 (segment (start 174.643814 91.9464) (end 152.5032 91.9464) (width 0.2) (layer "B.Cu") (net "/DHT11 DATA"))
 (segment (start 119.1514 93.3704) (end 119.1514 105.6894) (width 0.2) (layer "B.Cu") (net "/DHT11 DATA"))
 (segment (start 187.944 77.817786) (end 187.944 78.646214) (width 0.2) (layer "B.Cu") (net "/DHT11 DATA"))
 (segment (start 128.4018 108.9104) (end 126.483905 108.9104) (width 0.2) (layer "B.Cu") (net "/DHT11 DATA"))
 (segment (start 125.8618 91.631515) (end 140.261315 77.232) (width 0.2) (layer "B.Cu") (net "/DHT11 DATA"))
 (segment (start 119.1514 105.6894) (end 122.2756 108.8136) (width 0.2) (layer "B.Cu") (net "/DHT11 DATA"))
 (segment (start 187.358214 77.232) (end 187.944 77.817786) (width 0.2) (layer "B.Cu") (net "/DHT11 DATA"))
 (segment (start 187.944 78.646214) (end 174.643814 91.9464) (width 0.2) (layer "B.Cu") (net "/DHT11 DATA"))
 (segment (start 168.4782 91.694) (end 173.482 96.6978) (width 0.2) (layer "F.Cu") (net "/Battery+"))
 (segment (start 168.4782 90.5002) (end 168.4782 91.694) (width 0.2) (layer "F.Cu") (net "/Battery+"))
 (via (at 168.4782 90.5002) (size 0.6) (drill 0.3) (layers "F.Cu" "B.Cu") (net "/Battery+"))
 (segment (start 152.5824 86.614) (end 164.592 86.614) (width 0.2) (layer "B.Cu") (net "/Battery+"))
 (segment (start 164.592 86.614) (end 168.4782 90.5002) (width 0.2) (layer "B.Cu") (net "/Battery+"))
 (segment (start 161.7394 110.9804) (end 173.482 99.2378) (width 0.2) (layer "F.Cu") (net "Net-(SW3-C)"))
 (segment (start 161.7394 144.0688) (end 161.7394 110.9804) (width 0.2) (layer "F.Cu") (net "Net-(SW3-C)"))
 (segment (start 101.6 111.76) (end 130.6322 111.76) (width 0.2) (layer "B.Cu") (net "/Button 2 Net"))
 (segment (start 130.6322 111.76) (end 134.5438 107.8484) (width 0.2) (layer "B.Cu") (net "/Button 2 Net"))
 (segment (start 139.0396 79.0194) (end 126.9238 91.1352) (width 0.2) (layer "B.Cu") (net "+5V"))
 (segment (start 126.9238 91.1352) (end 126.9238 92.6084) (width 0.2) (layer "B.Cu") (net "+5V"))
 (segment (start 161.8742 79.0194) (end 139.0396 79.0194) (width 0.2) (layer "B.Cu") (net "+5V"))
 (segment (start 161.192156 146.0688) (end 160.8769 145.753544) (width 0.2) (layer "F.Cu") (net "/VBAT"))
 (segment (start 164.0144 146.0688) (end 161.192156 146.0688) (width 0.2) (layer "F.Cu") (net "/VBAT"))
 (segment (start 166.0144 144.0688) (end 164.0144 146.0688) (width 0.2) (layer "F.Cu") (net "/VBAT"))
 (segment (start 160.8769 145.753544) (end 160.8769 87.6367) (width 0.2) (layer "F.Cu") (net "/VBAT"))
 (segment (start 160.8769 87.6367) (end 169.4942 79.0194) (width 0.2) (layer "F.Cu") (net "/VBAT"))
 (segment (start 174.5488 79.0194) (end 174.9044 78.6638) (width 0.2) (layer "B.Cu") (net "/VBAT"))
 (segment (start 169.4942 79.0194) (end 174.5488 79.0194) (width 0.2) (layer "B.Cu") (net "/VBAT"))
 (segment (start 195.564 77.817786) (end 195.564 78.646214) (width 0.2) (layer "B.Cu") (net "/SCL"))
 (segment (start 128.3462 59.4676) (end 129.4962 58.3176) (width 0.2) (layer "B.Cu") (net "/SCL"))
 (segment (start 139.6238 114.2238) (end 139.6238 107.8484) (width 0.2) (layer "B.Cu") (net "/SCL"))
 (segment (start 176.159214 98.051) (end 171.189 98.051) (width 0.2) (layer "B.Cu") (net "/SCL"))
 (segment (start 194.578214 76.832) (end 195.564 77.817786) (width 0.2) (layer "B.Cu") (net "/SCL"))
 (segment (start 149.876946 76.832) (end 194.578214 76.832) (width 0.2) (layer "B.Cu") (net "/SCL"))
 (segment (start 171.189 98.051) (end 147.32 121.92) (width 0.2) (layer "B.Cu") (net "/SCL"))
 (segment (start 131.362546 58.3176) (end 149.876946 76.832) (width 0.2) (layer "B.Cu") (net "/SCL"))
 (segment (start 195.564 78.646214) (end 176.159214 98.051) (width 0.2) (layer "B.Cu") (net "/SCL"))
 (segment (start 147.32 121.92) (end 139.6238 114.2238) (width 0.2) (layer "B.Cu") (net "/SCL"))
 (segment (start 129.4962 58.3176) (end 131.362546 58.3176) (width 0.2) (layer "B.Cu") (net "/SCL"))
 (segment (start 97.809798 113.720101) (end 95.829899 115.7) (width 0.2) (layer "B.Cu") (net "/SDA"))
 (segment (start 95.829899 115.7) (end 94.670101 115.7) (width 0.2) (layer "B.Cu") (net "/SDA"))
 (segment (start 147.32 124.46) (end 137.0838 114.2238) (width 0.2) (layer "B.Cu") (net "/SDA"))
 (segment (start 137.0838 114.2238) (end 137.0838 107.8484) (width 0.2) (layer "B.Cu") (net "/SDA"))
 (segment (start 98.744872 79.843829) (end 110.509971 79.843829) (width 0.2) (layer "B.Cu") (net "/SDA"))
 (segment (start 91.7132 112.743099) (end 91.7132 86.875501) (width 0.2) (layer "B.Cu") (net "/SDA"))
 (segment (start 137.0838 107.8484) (end 131.212099 113.720101) (width 0.2) (layer "B.Cu") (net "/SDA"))
 (segment (start 110.509971 79.843829) (end 130.8862 59.4676) (width 0.2) (layer "B.Cu") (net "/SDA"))
 (segment (start 94.670101 115.7) (end 91.7132 112.743099) (width 0.2) (layer "B.Cu") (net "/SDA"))
 (segment (start 91.7132 86.875501) (end 98.744872 79.843829) (width 0.2) (layer "B.Cu") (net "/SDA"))
 (segment (start 131.212099 113.720101) (end 97.809798 113.720101) (width 0.2) (layer "B.Cu") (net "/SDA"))
 (segment (start 101.0276 132.7522) (end 102.7176 134.4422) (width 0.2) (layer "B.Cu") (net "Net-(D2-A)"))
 (segment (start 96.1376 132.7522) (end 101.0276 132.7522) (width 0.2) (layer "B.Cu") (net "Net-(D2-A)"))
 (segment (start 105.029 121.223871) (end 133.644471 92.6084) (width 0.2) (layer "F.Cu") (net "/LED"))
 (segment (start 133.644471 92.6084) (end 134.5438 92.6084) (width 0.2) (layer "F.Cu") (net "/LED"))
 (segment (start 105.029 127.762) (end 105.029 121.223871) (width 0.2) (layer "F.Cu") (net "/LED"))
 (via (at 105.029 127.762) (size 0.6) (drill 0.3) (layers "F.Cu" "B.Cu") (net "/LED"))
 (segment (start 88.5176 132.7522) (end 93.5078 127.762) (width 0.2) (layer "B.Cu") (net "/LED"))
 (segment (start 93.5078 127.762) (end 105.029 127.762) (width 0.2) (layer "B.Cu") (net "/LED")))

